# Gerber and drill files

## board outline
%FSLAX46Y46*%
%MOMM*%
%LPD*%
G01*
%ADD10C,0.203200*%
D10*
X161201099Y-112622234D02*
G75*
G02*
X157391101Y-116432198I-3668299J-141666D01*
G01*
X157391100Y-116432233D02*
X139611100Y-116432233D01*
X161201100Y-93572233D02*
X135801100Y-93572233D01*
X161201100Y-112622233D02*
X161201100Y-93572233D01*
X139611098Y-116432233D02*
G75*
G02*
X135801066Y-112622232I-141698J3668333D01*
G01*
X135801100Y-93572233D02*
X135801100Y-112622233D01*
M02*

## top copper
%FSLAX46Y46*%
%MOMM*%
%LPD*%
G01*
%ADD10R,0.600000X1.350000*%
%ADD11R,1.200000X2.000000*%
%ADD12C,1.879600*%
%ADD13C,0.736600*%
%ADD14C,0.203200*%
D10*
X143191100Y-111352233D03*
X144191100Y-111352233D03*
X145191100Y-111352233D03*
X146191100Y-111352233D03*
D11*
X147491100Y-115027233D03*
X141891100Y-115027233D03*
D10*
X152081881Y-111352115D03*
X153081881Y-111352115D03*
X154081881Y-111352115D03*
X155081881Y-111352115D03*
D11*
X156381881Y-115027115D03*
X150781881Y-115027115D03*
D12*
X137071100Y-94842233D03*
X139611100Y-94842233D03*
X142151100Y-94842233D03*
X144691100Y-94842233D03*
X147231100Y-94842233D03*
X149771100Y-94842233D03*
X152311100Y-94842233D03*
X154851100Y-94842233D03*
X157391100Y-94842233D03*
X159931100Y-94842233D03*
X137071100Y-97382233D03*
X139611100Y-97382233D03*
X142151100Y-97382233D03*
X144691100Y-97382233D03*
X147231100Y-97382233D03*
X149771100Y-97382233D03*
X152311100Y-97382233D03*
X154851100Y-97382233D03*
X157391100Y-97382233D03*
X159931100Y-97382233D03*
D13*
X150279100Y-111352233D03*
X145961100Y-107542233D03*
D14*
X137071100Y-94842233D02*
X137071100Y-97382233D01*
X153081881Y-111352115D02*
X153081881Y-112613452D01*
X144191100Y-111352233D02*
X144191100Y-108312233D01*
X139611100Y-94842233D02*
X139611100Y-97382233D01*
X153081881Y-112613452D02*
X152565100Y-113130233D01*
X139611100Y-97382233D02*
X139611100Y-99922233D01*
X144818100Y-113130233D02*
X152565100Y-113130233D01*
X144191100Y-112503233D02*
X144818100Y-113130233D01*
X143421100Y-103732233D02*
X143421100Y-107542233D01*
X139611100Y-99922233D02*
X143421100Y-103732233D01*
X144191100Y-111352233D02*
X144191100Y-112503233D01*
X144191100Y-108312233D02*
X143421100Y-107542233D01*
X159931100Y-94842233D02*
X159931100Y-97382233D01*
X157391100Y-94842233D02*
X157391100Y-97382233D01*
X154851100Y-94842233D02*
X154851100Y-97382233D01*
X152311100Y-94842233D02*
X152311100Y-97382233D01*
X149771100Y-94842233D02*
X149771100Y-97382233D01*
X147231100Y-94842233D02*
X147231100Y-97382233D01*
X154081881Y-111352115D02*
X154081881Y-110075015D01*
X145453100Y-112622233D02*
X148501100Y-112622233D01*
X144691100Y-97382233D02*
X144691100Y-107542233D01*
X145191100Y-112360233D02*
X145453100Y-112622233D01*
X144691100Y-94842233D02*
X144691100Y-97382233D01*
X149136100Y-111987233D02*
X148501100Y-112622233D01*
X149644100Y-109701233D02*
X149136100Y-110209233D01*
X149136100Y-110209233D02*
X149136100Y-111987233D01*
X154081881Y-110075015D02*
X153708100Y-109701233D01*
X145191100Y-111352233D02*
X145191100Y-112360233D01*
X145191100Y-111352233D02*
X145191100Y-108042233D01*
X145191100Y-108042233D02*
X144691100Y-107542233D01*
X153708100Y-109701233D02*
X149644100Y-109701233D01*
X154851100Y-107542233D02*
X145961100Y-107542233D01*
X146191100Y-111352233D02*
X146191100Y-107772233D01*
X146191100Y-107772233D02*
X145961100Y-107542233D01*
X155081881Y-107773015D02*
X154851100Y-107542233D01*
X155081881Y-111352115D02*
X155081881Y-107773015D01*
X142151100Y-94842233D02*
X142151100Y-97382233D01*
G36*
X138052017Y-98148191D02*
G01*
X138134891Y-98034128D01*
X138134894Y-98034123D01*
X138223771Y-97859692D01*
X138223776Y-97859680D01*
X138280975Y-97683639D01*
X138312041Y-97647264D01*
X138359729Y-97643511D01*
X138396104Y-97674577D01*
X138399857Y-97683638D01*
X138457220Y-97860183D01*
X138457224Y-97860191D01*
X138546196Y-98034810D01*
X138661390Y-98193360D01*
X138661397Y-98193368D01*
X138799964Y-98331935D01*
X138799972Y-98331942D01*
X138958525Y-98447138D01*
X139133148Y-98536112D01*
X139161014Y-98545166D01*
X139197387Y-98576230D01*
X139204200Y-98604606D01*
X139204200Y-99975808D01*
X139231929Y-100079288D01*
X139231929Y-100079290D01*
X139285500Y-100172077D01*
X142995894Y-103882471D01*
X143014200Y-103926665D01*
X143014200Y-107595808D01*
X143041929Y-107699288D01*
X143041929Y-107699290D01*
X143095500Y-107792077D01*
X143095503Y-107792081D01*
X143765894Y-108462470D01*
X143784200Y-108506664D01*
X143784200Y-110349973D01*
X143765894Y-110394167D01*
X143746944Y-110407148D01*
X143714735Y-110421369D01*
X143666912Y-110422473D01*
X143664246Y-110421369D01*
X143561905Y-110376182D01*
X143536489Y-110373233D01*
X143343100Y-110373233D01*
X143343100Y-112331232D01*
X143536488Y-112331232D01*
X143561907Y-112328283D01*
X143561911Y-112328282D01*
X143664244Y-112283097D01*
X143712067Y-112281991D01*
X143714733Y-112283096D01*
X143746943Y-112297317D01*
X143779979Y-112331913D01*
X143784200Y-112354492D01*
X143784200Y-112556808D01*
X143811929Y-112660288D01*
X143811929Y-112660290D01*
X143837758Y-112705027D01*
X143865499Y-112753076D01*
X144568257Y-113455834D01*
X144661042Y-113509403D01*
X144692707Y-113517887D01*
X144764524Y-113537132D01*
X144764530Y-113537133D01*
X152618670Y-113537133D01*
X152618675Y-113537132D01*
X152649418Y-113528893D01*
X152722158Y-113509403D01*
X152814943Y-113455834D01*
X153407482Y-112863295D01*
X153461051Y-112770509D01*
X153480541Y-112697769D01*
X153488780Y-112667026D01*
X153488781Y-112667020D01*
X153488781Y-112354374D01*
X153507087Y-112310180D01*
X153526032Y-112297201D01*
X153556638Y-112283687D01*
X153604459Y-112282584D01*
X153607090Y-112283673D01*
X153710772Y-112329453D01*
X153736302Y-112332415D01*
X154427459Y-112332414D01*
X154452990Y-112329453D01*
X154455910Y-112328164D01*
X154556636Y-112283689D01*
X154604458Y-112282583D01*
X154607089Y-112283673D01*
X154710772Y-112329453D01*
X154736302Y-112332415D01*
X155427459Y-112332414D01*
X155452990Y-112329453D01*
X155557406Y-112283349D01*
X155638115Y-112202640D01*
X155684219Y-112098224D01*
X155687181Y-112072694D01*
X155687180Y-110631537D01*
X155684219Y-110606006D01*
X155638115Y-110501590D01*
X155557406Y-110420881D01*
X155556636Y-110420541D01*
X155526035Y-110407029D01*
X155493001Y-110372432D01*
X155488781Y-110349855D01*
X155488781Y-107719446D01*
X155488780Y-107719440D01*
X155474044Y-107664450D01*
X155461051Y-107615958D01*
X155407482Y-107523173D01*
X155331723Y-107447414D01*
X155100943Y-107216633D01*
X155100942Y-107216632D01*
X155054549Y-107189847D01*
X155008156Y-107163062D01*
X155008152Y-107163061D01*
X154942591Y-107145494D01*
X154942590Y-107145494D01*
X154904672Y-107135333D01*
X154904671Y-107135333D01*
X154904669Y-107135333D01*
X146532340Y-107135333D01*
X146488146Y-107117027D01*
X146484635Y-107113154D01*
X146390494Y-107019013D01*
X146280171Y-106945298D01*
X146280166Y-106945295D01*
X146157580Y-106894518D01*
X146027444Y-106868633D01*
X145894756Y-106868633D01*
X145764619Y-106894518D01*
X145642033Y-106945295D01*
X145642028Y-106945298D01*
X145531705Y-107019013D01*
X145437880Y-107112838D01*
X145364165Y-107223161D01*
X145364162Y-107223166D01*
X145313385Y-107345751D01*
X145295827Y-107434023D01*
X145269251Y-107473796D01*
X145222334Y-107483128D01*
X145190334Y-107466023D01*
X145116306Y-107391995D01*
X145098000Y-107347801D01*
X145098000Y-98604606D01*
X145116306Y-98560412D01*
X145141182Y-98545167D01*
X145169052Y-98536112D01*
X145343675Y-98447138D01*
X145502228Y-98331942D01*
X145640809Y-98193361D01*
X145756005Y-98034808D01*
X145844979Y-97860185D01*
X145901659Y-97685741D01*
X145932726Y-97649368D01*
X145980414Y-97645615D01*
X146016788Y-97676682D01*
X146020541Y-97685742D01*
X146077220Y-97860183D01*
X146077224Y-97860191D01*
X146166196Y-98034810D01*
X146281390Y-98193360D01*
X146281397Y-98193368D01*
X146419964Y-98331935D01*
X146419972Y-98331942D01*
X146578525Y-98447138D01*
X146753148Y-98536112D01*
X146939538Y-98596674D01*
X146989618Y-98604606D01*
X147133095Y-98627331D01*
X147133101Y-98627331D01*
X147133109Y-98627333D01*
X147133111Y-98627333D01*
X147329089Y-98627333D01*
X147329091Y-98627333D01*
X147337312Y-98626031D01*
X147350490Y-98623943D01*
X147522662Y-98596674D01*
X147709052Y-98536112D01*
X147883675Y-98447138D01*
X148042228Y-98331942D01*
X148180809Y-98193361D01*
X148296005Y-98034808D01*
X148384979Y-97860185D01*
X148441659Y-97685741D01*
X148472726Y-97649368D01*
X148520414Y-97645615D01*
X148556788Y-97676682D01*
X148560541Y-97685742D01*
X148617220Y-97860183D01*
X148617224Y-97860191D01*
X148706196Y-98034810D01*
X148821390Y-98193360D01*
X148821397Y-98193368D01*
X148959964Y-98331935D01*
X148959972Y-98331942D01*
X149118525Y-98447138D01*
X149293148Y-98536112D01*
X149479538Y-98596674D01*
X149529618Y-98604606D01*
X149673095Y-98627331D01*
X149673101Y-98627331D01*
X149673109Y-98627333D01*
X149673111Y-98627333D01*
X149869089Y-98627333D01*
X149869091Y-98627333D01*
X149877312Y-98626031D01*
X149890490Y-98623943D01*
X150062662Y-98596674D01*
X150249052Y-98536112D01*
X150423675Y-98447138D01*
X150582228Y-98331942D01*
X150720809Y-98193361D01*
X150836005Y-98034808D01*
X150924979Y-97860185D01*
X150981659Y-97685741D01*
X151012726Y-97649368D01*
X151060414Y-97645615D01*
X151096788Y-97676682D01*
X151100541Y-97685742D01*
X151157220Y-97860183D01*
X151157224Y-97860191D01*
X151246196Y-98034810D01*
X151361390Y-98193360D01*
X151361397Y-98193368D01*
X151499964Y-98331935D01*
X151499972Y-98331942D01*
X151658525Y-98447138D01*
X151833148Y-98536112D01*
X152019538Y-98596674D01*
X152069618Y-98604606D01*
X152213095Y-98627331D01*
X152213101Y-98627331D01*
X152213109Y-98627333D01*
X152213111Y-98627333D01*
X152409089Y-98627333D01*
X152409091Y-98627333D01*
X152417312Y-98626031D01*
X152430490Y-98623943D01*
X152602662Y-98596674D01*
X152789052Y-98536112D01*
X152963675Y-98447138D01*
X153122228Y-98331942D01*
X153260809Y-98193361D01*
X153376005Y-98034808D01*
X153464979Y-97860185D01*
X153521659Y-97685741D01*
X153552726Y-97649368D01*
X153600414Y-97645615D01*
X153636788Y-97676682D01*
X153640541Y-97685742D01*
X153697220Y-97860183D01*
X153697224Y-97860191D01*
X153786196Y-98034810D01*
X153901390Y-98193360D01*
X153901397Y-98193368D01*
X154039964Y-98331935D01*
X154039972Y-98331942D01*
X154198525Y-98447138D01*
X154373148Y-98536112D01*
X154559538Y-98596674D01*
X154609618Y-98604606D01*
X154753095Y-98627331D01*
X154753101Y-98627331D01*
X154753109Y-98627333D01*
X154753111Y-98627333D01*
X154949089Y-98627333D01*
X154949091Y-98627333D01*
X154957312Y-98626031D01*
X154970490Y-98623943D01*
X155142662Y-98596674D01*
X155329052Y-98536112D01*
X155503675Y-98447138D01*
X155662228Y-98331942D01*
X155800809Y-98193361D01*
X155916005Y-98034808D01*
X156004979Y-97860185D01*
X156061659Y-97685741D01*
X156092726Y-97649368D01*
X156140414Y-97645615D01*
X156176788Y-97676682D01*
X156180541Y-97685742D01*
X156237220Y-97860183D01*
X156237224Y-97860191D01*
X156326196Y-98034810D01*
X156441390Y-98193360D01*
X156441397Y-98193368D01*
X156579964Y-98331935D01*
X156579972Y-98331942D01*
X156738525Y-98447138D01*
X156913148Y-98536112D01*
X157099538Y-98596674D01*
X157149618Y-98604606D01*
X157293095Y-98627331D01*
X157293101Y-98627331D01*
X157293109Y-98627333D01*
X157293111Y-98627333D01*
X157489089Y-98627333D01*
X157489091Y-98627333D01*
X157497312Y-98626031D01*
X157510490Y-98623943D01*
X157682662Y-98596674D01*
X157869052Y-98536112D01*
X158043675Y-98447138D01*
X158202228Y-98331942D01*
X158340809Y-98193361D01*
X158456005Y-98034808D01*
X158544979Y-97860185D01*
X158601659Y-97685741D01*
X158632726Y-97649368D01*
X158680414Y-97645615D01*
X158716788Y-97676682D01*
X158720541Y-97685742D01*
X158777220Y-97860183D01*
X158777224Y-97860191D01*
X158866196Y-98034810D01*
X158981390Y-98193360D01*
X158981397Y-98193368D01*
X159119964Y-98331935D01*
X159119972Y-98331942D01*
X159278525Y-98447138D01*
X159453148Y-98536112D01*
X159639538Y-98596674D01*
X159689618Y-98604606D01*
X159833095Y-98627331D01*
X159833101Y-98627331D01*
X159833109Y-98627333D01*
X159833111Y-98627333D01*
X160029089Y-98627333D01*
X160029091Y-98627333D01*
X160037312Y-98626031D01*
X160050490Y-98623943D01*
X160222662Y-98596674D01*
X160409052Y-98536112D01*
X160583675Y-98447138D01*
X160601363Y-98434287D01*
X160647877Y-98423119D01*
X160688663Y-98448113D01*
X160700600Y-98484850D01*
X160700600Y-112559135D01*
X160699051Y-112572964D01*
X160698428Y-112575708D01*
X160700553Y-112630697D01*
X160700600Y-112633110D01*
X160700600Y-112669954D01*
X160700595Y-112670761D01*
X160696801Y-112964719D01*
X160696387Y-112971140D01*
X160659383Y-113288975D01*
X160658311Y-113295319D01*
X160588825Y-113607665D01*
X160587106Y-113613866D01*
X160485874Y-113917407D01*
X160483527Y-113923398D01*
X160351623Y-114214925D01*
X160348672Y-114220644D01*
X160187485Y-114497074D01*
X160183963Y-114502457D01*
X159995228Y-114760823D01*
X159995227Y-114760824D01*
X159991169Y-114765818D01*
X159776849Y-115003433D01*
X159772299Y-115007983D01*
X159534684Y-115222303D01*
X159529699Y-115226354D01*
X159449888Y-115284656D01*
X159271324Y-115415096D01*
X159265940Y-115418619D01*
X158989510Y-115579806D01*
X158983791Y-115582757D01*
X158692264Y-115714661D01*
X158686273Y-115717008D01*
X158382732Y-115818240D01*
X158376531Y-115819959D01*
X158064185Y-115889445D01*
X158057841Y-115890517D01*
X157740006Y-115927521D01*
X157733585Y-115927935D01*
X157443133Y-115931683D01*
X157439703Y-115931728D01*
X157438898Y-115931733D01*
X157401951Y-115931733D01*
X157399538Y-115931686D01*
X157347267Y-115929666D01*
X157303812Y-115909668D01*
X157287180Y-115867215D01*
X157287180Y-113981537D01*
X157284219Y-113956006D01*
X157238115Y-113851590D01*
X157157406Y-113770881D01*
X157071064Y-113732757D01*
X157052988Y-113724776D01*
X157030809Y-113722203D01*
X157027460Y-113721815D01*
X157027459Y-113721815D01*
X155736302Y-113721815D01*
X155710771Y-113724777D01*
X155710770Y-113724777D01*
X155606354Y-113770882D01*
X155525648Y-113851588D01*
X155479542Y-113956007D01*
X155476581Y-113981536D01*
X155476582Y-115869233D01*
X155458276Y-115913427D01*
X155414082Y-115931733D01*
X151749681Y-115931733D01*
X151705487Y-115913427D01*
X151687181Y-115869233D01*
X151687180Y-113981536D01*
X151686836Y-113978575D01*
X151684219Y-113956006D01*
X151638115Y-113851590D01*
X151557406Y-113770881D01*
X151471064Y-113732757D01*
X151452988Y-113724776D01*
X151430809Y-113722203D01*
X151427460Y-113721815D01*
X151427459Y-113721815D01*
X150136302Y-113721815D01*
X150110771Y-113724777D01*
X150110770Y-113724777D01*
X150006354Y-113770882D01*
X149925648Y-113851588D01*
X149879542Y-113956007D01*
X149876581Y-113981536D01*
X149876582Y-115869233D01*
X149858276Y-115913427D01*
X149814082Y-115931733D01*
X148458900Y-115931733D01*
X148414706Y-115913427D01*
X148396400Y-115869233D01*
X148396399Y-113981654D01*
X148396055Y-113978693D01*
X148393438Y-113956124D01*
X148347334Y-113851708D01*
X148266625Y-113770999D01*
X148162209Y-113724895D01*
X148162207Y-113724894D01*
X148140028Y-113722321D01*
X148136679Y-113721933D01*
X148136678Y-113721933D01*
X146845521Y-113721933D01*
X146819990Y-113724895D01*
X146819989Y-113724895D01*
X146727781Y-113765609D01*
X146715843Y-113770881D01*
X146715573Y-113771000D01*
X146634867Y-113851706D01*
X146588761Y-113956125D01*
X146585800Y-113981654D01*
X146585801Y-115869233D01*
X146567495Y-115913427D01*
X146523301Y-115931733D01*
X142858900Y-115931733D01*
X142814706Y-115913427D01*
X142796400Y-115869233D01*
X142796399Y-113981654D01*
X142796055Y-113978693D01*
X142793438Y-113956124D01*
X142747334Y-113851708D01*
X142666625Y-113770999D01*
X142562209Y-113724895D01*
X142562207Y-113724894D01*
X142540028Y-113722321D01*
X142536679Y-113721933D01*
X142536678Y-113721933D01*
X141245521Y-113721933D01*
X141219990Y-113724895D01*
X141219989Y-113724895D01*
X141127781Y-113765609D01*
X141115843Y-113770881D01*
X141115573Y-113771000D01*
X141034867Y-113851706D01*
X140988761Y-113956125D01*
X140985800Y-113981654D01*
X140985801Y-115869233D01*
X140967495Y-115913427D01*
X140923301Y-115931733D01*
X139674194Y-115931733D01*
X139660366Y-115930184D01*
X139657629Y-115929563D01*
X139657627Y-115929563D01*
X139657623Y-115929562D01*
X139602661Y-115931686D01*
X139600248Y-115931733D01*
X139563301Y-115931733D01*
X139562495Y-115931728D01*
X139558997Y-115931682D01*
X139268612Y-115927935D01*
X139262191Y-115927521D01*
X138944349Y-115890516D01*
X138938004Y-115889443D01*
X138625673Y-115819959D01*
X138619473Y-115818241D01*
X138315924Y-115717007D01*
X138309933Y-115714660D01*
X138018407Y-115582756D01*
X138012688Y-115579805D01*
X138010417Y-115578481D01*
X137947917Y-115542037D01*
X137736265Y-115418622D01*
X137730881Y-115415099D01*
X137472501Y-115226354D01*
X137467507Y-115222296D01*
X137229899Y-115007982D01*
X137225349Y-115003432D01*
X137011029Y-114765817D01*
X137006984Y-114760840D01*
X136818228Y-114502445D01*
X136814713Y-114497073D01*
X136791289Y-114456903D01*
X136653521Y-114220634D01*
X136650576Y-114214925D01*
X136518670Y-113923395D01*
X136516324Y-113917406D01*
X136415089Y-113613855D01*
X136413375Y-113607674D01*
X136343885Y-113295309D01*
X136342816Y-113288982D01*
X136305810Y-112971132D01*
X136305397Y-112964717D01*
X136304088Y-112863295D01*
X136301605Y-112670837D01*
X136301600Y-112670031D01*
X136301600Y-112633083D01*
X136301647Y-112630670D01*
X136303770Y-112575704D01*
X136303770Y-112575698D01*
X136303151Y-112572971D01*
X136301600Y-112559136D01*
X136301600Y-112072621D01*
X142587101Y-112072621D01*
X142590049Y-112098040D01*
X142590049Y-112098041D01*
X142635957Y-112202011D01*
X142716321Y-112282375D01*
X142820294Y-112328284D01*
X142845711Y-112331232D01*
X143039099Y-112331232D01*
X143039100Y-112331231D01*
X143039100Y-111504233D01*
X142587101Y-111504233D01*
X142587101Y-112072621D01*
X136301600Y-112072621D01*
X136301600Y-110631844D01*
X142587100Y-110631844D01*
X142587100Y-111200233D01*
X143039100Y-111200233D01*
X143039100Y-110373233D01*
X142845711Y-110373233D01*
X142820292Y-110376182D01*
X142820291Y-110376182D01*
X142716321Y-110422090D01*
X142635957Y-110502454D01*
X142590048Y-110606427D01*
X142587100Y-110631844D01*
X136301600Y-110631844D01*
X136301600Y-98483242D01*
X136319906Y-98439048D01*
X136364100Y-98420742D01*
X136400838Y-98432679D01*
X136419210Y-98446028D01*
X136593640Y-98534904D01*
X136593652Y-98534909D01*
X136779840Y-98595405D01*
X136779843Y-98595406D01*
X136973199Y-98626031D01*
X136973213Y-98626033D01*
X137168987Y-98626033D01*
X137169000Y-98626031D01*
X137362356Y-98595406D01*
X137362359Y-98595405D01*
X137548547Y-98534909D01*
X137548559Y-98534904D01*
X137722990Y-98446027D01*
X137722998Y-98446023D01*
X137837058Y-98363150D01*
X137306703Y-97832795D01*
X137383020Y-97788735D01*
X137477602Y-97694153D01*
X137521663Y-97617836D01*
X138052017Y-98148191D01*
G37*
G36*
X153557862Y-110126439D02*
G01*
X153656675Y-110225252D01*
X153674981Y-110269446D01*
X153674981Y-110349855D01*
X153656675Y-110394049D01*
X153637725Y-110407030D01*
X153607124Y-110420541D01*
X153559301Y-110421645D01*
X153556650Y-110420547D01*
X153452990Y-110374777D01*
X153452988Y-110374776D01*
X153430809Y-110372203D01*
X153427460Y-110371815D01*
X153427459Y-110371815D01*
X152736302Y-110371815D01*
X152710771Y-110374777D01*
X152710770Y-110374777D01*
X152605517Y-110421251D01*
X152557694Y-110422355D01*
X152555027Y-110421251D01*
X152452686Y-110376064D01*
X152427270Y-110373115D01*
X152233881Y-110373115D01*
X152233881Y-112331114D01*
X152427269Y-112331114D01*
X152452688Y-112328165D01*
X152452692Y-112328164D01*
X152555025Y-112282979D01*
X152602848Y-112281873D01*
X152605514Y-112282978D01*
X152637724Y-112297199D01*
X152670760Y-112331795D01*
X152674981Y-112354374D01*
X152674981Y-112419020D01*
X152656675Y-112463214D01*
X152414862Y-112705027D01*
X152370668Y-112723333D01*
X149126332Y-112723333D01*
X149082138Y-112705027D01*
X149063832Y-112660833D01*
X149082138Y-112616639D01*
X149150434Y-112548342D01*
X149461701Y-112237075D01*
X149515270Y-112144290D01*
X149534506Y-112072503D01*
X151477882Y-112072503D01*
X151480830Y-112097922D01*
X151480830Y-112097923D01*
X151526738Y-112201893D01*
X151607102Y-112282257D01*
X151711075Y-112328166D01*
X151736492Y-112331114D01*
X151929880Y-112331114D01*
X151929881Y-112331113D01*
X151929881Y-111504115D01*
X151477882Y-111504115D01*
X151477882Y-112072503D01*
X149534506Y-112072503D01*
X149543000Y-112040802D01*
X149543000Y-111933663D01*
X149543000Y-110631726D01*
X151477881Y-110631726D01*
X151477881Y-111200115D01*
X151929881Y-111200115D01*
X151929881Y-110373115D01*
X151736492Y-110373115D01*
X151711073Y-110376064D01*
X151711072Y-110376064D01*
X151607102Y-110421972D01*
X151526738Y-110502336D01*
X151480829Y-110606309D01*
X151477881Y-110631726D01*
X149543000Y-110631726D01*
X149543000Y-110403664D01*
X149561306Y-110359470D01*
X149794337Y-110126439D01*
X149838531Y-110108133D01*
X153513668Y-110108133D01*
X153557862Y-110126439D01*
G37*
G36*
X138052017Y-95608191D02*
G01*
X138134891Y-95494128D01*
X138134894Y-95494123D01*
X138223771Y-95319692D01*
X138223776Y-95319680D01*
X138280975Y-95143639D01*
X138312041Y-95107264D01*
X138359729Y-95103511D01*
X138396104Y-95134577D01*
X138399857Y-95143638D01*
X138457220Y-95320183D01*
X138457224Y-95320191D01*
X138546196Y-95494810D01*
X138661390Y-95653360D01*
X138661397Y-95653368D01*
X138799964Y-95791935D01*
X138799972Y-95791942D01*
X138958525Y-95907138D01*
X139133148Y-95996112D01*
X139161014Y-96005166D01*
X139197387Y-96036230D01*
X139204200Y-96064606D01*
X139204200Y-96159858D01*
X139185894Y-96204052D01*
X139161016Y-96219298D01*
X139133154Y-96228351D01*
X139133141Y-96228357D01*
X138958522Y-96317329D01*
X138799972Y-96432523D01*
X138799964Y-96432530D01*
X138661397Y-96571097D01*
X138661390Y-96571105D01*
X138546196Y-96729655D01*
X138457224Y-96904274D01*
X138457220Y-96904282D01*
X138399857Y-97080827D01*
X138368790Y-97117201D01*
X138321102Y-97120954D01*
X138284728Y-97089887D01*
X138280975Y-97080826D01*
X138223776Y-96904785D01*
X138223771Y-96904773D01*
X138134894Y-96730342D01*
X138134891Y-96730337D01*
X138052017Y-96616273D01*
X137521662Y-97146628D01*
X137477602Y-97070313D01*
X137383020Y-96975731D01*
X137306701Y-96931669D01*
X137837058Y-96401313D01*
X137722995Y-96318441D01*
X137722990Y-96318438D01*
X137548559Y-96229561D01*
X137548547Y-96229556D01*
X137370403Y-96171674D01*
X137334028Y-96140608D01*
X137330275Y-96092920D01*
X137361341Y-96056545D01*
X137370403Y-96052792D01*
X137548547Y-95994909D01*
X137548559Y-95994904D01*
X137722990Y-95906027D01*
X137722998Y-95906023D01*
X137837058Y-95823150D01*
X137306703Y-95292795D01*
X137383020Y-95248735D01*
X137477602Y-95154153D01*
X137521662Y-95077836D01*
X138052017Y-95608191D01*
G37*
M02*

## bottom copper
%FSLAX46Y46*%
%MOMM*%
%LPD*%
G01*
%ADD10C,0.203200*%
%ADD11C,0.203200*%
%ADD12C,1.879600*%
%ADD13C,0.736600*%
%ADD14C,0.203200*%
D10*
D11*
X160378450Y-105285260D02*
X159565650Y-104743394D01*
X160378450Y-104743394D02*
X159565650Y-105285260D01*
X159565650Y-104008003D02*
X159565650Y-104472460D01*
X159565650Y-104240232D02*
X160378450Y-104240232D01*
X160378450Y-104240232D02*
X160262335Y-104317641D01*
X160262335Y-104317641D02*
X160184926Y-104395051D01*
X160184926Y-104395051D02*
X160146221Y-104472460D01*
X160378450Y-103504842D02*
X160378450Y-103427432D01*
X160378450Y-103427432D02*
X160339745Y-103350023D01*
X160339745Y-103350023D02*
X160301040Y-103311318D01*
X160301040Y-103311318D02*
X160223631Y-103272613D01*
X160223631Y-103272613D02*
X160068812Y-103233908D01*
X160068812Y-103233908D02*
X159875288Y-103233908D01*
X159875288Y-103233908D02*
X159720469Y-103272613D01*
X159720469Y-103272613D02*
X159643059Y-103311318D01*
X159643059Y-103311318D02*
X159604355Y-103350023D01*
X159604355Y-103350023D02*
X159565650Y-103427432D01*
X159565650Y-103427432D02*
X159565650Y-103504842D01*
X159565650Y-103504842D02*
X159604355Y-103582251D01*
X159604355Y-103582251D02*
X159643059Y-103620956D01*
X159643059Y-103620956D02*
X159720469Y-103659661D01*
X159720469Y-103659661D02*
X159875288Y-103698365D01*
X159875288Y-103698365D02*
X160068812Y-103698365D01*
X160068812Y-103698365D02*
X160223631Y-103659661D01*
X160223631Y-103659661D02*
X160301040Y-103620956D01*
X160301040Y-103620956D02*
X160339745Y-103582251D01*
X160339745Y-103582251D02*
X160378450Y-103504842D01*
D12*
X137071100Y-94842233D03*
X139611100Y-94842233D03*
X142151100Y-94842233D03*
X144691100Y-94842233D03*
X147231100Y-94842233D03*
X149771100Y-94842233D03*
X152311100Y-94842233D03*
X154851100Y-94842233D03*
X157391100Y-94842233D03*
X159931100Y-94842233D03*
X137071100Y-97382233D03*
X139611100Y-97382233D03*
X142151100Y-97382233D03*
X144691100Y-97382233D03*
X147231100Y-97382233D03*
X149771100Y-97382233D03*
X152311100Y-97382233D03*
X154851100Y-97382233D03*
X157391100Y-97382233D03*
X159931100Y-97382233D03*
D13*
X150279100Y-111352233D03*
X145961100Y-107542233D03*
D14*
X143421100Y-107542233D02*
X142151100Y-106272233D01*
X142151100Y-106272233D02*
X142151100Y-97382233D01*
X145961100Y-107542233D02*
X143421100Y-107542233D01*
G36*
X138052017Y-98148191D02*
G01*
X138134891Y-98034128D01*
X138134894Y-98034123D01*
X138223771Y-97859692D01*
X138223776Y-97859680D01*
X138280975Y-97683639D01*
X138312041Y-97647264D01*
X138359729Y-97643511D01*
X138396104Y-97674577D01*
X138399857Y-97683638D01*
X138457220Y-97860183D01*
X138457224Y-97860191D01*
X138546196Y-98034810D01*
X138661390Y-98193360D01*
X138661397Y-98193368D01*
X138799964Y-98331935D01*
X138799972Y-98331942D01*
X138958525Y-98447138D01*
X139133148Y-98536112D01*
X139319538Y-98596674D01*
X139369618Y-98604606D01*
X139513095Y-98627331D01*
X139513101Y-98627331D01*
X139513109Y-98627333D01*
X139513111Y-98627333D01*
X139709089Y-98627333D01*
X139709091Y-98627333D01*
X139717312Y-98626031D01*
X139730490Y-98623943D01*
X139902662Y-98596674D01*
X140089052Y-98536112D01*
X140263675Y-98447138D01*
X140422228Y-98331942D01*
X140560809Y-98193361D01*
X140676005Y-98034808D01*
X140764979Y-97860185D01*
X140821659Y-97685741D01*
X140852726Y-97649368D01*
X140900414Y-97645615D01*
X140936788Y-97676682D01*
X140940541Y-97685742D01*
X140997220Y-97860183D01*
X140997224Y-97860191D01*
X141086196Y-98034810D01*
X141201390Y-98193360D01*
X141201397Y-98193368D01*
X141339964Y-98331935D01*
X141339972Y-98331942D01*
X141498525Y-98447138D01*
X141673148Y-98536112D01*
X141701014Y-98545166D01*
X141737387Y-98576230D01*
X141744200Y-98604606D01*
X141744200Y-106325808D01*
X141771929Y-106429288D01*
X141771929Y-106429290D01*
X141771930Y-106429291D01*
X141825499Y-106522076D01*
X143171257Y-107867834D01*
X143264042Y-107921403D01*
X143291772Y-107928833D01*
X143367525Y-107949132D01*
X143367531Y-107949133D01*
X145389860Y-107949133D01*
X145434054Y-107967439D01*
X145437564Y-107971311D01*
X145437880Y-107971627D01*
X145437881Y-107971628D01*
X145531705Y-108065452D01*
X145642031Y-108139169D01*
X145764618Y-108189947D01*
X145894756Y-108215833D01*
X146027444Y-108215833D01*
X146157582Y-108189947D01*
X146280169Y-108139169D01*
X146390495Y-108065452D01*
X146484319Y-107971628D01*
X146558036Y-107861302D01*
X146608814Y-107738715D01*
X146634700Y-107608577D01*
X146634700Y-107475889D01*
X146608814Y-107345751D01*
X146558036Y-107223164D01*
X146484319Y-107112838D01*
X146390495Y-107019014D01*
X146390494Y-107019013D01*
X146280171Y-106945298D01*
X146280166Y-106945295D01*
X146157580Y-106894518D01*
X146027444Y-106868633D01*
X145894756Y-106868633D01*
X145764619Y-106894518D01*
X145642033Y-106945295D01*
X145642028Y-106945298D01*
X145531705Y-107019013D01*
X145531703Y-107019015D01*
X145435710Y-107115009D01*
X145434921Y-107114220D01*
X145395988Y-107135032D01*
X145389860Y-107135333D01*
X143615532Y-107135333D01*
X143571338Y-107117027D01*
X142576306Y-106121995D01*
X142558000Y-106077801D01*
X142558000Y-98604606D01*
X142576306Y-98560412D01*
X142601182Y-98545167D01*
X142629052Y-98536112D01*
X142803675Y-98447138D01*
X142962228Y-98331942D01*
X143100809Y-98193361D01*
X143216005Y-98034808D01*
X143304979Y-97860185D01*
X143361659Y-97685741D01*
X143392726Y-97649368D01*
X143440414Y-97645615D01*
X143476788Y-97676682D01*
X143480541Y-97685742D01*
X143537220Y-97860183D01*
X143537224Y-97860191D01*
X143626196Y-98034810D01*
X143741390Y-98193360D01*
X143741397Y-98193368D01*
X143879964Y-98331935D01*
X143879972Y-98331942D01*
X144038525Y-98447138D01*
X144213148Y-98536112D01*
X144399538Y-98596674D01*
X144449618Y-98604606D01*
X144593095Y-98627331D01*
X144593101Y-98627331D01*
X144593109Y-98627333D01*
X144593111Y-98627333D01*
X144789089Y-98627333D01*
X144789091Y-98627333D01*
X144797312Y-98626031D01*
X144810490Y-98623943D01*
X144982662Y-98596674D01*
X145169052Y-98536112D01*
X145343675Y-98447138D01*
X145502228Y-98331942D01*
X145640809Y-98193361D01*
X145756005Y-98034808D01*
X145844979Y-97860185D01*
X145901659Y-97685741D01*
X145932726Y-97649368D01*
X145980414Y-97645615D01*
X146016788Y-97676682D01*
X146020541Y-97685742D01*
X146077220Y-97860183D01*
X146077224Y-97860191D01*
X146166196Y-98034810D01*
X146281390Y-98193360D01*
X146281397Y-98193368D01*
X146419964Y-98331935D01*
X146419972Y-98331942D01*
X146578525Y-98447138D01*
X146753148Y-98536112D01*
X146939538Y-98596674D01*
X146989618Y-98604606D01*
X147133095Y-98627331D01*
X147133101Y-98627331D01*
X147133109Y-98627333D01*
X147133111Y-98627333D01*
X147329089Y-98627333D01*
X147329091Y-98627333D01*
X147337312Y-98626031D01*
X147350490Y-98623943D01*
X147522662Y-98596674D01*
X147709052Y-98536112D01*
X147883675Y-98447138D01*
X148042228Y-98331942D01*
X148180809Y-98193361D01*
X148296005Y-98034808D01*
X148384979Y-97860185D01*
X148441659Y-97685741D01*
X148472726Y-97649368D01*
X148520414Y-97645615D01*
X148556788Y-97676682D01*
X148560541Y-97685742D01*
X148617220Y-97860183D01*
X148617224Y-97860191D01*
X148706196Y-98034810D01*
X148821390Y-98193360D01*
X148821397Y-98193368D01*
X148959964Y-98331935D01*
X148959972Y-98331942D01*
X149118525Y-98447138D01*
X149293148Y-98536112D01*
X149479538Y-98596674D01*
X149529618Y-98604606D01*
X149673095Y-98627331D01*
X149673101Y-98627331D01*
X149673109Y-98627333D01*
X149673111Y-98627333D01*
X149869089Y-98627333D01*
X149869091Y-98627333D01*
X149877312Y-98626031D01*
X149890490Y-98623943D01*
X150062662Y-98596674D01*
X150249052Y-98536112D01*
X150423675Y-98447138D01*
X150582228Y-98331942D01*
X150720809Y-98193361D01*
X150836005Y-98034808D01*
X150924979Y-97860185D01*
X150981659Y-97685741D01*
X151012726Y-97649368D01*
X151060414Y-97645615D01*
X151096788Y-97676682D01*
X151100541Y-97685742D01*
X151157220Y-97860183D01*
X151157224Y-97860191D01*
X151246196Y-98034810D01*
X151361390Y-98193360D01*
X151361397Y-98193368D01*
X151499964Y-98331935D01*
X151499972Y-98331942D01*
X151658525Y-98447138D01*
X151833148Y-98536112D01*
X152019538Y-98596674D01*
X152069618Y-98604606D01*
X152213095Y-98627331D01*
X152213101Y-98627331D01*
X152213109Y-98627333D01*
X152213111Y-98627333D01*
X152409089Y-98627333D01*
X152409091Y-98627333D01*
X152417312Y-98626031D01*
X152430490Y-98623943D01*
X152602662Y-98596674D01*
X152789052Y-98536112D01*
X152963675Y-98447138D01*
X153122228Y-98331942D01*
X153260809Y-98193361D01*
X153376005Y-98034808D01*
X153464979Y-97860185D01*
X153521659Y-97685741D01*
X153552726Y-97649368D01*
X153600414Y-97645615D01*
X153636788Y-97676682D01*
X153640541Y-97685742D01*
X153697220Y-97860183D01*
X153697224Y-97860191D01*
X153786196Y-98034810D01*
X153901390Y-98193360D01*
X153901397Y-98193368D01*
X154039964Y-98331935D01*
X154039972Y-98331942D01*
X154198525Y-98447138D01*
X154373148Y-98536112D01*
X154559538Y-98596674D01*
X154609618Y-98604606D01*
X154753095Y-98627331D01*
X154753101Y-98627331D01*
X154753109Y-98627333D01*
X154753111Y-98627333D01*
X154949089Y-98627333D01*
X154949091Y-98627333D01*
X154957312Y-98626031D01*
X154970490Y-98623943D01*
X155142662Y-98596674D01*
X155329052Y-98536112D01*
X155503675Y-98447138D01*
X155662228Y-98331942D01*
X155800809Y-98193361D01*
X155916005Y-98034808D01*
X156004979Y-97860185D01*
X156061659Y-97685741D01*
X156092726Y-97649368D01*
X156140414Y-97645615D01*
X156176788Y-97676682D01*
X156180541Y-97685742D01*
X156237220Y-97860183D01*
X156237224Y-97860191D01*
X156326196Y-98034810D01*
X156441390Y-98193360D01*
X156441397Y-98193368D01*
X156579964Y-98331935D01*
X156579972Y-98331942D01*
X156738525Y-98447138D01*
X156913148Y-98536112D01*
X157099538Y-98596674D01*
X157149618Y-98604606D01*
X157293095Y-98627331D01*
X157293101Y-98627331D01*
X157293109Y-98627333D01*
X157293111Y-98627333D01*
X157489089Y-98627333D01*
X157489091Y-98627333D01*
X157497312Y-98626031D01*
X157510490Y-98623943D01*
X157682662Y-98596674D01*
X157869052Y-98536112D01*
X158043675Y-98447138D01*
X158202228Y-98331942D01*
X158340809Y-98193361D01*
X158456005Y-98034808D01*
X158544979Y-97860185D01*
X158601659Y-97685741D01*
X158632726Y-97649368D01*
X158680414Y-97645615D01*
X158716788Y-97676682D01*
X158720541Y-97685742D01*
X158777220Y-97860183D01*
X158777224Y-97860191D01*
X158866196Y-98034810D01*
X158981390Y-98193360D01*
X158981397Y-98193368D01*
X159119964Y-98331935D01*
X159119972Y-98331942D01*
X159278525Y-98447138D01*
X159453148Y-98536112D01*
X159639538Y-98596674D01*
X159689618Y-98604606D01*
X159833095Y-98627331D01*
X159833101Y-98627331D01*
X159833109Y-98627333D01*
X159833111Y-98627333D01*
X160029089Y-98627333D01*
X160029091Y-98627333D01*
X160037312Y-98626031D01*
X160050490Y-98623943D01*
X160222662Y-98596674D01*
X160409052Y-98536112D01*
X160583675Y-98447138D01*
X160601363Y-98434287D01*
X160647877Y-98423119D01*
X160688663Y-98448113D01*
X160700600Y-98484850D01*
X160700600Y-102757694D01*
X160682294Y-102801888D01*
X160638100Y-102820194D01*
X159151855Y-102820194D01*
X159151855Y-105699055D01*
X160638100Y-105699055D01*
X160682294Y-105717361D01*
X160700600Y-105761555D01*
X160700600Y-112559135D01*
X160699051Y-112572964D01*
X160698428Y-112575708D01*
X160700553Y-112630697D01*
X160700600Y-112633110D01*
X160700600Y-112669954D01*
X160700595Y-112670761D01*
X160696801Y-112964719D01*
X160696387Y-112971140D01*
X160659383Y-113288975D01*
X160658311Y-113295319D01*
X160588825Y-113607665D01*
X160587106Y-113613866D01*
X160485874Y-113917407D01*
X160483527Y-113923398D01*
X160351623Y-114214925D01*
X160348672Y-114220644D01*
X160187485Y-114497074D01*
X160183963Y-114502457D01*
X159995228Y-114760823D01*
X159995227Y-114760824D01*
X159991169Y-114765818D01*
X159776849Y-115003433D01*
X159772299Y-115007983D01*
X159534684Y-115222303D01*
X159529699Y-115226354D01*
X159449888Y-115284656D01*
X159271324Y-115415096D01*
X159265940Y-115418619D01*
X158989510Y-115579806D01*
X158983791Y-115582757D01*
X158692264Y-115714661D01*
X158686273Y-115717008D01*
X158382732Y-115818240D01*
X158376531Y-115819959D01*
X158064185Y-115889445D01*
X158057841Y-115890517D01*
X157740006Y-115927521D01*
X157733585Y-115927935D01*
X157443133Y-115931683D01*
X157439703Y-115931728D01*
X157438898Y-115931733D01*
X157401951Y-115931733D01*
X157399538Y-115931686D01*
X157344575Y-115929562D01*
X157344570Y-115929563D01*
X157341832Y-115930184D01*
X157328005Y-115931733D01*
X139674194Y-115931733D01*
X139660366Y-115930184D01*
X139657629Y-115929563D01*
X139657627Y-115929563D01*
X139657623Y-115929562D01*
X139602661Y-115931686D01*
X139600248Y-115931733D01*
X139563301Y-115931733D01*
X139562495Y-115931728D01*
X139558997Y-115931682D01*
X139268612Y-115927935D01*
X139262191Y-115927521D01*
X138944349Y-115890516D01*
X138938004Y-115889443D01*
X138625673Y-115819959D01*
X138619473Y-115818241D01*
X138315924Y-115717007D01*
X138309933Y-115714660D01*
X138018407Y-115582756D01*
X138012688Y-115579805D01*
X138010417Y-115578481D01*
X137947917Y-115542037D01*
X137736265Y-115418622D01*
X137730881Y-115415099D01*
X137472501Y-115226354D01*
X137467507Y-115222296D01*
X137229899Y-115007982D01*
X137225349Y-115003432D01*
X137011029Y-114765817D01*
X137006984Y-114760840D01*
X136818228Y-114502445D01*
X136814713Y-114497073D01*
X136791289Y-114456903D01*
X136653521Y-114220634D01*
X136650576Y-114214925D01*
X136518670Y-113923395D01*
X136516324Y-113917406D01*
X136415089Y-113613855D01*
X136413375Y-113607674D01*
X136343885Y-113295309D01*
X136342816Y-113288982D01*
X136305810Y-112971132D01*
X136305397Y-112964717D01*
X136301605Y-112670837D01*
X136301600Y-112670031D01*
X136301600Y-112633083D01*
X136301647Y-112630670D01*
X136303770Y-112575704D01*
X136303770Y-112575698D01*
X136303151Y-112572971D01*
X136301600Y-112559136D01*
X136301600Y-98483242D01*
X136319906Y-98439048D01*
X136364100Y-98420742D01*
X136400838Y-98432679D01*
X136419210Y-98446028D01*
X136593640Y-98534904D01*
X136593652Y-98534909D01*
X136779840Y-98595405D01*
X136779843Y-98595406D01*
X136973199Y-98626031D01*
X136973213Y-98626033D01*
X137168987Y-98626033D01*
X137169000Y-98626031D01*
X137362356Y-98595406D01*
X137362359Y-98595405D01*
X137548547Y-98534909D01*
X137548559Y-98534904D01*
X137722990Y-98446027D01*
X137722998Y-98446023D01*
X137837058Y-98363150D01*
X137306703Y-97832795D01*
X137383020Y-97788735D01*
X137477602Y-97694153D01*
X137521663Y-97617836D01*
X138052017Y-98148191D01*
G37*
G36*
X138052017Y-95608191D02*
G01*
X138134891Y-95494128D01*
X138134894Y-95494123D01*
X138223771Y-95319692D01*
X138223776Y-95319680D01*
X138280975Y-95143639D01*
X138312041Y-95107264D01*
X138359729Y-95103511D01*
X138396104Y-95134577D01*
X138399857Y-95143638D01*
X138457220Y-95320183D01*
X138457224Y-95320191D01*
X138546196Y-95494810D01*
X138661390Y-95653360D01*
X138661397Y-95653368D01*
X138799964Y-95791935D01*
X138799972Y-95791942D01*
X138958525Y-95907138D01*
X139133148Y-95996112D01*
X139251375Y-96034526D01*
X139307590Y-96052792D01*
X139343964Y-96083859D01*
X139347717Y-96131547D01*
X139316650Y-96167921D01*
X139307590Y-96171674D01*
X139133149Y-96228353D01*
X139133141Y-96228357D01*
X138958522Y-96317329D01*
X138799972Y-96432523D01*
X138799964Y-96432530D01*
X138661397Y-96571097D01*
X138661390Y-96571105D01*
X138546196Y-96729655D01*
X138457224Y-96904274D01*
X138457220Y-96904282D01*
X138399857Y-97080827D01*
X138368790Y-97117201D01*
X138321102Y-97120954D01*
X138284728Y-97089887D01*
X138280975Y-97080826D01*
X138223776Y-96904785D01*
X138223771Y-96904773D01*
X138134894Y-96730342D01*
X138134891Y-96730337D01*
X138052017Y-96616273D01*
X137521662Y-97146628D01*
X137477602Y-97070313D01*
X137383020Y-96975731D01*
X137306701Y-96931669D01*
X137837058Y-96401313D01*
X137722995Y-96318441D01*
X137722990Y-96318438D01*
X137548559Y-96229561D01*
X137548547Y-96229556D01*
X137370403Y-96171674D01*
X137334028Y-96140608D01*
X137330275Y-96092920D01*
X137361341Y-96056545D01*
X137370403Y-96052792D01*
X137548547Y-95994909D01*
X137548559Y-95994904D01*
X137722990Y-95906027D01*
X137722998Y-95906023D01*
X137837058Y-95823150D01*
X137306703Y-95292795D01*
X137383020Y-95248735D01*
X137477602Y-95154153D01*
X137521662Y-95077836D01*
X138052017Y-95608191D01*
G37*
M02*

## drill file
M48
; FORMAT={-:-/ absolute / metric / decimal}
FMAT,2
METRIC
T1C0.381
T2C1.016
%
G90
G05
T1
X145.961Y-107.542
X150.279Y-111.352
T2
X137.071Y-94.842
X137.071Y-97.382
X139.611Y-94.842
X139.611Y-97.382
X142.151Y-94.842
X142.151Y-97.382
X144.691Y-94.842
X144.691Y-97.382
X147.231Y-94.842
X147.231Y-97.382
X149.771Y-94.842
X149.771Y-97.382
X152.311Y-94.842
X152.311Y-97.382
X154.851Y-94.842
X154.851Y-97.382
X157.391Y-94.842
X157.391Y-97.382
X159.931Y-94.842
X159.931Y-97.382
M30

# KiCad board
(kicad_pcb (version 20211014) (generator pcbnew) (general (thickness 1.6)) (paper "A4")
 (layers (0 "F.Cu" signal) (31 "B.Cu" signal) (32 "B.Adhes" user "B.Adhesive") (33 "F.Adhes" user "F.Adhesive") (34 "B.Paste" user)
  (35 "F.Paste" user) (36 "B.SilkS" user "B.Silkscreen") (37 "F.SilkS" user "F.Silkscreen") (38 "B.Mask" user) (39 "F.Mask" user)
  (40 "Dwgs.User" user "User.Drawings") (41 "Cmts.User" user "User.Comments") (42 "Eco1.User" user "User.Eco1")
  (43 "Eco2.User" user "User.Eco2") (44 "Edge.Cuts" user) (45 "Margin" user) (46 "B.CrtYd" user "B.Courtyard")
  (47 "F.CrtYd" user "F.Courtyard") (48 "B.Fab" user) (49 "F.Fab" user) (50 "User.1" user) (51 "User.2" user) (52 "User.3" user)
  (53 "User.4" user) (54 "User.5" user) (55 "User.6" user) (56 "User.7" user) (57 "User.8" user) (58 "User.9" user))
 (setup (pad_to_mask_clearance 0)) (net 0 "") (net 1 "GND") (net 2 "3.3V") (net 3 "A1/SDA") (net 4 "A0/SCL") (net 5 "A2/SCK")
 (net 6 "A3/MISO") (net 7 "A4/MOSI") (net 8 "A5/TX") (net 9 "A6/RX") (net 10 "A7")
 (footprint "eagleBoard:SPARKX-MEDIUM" (layer "F.Cu") (at 138.3411 108.812233 90)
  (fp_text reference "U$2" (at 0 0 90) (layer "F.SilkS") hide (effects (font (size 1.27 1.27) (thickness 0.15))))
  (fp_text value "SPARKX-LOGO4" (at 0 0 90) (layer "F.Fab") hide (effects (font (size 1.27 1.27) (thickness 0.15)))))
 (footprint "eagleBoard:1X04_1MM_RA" (layer "F.Cu") (at 144.6911 111.352233)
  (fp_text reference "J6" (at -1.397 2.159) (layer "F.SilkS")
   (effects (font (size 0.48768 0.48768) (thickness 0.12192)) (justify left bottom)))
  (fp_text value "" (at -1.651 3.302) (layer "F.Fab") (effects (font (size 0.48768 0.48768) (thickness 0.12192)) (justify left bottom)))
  (pad "1" smd rect (at -1.5 0) (size 0.6 1.35) (layers "F.Cu" "F.Paste" "F.Mask") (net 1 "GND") (solder_mask_margin 0.1016))
  (pad "2" smd rect (at -0.5 0) (size 0.6 1.35) (layers "F.Cu" "F.Paste" "F.Mask") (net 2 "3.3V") (solder_mask_margin 0.1016))
  (pad "3" smd rect (at 0.5 0) (size 0.6 1.35) (layers "F.Cu" "F.Paste" "F.Mask") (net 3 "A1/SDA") (solder_mask_margin 0.1016))
  (pad "4" smd rect (at 1.5 0) (size 0.6 1.35) (layers "F.Cu" "F.Paste" "F.Mask") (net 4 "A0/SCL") (solder_mask_margin 0.1016))
  (pad "NC1" smd rect (at 2.8 3.675) (size 1.2 2) (layers "F.Cu" "F.Paste" "F.Mask") (solder_mask_margin 0.1016))
  (pad "NC2" smd rect (at -2.8 3.675) (size 1.2 2) (layers "F.Cu" "F.Paste" "F.Mask") (solder_mask_margin 0.1016)))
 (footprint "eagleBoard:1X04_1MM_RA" (layer "F.Cu") (at 153.581881 111.352115)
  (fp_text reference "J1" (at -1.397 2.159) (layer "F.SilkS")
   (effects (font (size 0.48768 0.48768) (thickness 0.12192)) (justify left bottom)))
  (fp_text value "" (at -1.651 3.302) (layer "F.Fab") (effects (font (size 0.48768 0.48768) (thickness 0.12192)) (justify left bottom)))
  (pad "1" smd rect (at -1.5 0) (size 0.6 1.35) (layers "F.Cu" "F.Paste" "F.Mask") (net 1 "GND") (solder_mask_margin 0.1016))
  (pad "2" smd rect (at -0.5 0) (size 0.6 1.35) (layers "F.Cu" "F.Paste" "F.Mask") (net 2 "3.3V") (solder_mask_margin 0.1016))
  (pad "3" smd rect (at 0.5 0) (size 0.6 1.35) (layers "F.Cu" "F.Paste" "F.Mask") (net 3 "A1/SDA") (solder_mask_margin 0.1016))
  (pad "4" smd rect (at 1.5 0) (size 0.6 1.35) (layers "F.Cu" "F.Paste" "F.Mask") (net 4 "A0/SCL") (solder_mask_margin 0.1016))
  (pad "NC1" smd rect (at 2.8 3.675) (size 1.2 2) (layers "F.Cu" "F.Paste" "F.Mask") (solder_mask_margin 0.1016))
  (pad "NC2" smd rect (at -2.8 3.675) (size 1.2 2) (layers "F.Cu" "F.Paste" "F.Mask") (solder_mask_margin 0.1016)))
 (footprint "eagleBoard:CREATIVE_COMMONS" (layer "F.Cu") (at 126.9111 140.562233)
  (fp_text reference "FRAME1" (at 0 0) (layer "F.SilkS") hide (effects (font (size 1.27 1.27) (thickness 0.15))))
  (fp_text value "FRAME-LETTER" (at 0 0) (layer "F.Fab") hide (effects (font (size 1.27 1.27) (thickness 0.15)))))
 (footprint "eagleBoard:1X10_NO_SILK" (layer "F.Cu") (at 137.0711 94.842233)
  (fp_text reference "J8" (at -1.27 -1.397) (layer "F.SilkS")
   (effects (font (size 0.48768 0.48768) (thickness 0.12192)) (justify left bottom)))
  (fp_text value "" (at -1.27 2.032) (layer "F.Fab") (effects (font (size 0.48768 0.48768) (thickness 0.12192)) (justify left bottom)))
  (pad "1" thru_hole circle (at 0 0 90) (size 1.8796 1.8796) (drill 1.016) (layers *.Cu *.Mask) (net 1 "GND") (solder_mask_margin 0.1016))
  (pad "2" thru_hole circle (at 2.54 0 90) (size 1.8796 1.8796) (drill 1.016) (layers *.Cu *.Mask) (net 2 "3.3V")
   (solder_mask_margin 0.1016))
  (pad "3" thru_hole circle (at 5.08 0 90) (size 1.8796 1.8796) (drill 1.016) (layers *.Cu *.Mask) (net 4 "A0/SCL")
   (solder_mask_margin 0.1016))
  (pad "4" thru_hole circle (at 7.62 0 90) (size 1.8796 1.8796) (drill 1.016) (layers *.Cu *.Mask) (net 3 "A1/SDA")
   (solder_mask_margin 0.1016))
  (pad "5" thru_hole circle (at 10.16 0 90) (size 1.8796 1.8796) (drill 1.016) (layers *.Cu *.Mask) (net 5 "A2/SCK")
   (solder_mask_margin 0.1016))
  (pad "6" thru_hole circle (at 12.7 0 90) (size 1.8796 1.8796) (drill 1.016) (layers *.Cu *.Mask) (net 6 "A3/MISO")
   (solder_mask_margin 0.1016))
  (pad "7" thru_hole circle (at 15.24 0 90) (size 1.8796 1.8796) (drill 1.016) (layers *.Cu *.Mask) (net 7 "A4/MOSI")
   (solder_mask_margin 0.1016))
  (pad "8" thru_hole circle (at 17.78 0 90) (size 1.8796 1.8796) (drill 1.016) (layers *.Cu *.Mask) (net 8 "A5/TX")
   (solder_mask_margin 0.1016))
  (pad "9" thru_hole circle (at 20.32 0 90) (size 1.8796 1.8796) (drill 1.016) (layers *.Cu *.Mask) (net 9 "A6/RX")
   (solder_mask_margin 0.1016))
  (pad "10" thru_hole circle (at 22.86 0 90) (size 1.8796 1.8796) (drill 1.016) (layers *.Cu *.Mask) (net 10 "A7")
   (solder_mask_margin 0.1016)))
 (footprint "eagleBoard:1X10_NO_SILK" (layer "F.Cu") (at 137.0711 97.382233)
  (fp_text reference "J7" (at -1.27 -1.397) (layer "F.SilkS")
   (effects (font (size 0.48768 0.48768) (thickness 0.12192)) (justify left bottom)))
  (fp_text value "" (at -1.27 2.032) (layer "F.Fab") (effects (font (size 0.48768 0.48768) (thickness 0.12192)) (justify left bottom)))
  (pad "1" thru_hole circle (at 0 0 90) (size 1.8796 1.8796) (drill 1.016) (layers *.Cu *.Mask) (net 1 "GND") (solder_mask_margin 0.1016))
  (pad "2" thru_hole circle (at 2.54 0 90) (size 1.8796 1.8796) (drill 1.016) (layers *.Cu *.Mask) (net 2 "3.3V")
   (solder_mask_margin 0.1016))
  (pad "3" thru_hole circle (at 5.08 0 90) (size 1.8796 1.8796) (drill 1.016) (layers *.Cu *.Mask) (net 4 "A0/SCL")
   (solder_mask_margin 0.1016))
  (pad "4" thru_hole circle (at 7.62 0 90) (size 1.8796 1.8796) (drill 1.016) (layers *.Cu *.Mask) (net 3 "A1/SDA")
   (solder_mask_margin 0.1016))
  (pad "5" thru_hole circle (at 10.16 0 90) (size 1.8796 1.8796) (drill 1.016) (layers *.Cu *.Mask) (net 5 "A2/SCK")
   (solder_mask_margin 0.1016))
  (pad "6" thru_hole circle (at 12.7 0 90) (size 1.8796 1.8796) (drill 1.016) (layers *.Cu *.Mask) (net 6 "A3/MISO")
   (solder_mask_margin 0.1016))
  (pad "7" thru_hole circle (at 15.24 0 90) (size 1.8796 1.8796) (drill 1.016) (layers *.Cu *.Mask) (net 7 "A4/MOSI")
   (solder_mask_margin 0.1016))
  (pad "8" thru_hole circle (at 17.78 0 90) (size 1.8796 1.8796) (drill 1.016) (layers *.Cu *.Mask) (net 8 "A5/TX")
   (solder_mask_margin 0.1016))
  (pad "9" thru_hole circle (at 20.32 0 90) (size 1.8796 1.8796) (drill 1.016) (layers *.Cu *.Mask) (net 9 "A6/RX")
   (solder_mask_margin 0.1016))
  (pad "10" thru_hole circle (at 22.86 0 90) (size 1.8796 1.8796) (drill 1.016) (layers *.Cu *.Mask) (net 10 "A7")
   (solder_mask_margin 0.1016)))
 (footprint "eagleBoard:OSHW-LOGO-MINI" (layer "B.Cu") (at 159.4231 112.114233 180)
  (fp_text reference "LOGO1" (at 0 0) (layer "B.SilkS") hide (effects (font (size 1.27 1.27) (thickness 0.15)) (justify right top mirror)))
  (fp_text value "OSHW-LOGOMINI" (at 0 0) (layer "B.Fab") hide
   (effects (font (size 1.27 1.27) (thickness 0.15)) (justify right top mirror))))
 (gr_arc (start 161.201099 112.622234) (mid 160.128599 115.359733) (end 157.3911 116.432233) (layer "Edge.Cuts") (width 0.2032))
 (gr_line (start 157.3911 116.432233) (end 139.6111 116.432233) (layer "Edge.Cuts") (width 0.2032))
 (gr_line (start 161.2011 93.572233) (end 135.8011 93.572233) (layer "Edge.Cuts") (width 0.2032))
 (gr_line (start 161.2011 112.622233) (end 161.2011 93.572233) (layer "Edge.Cuts") (width 0.2032))
 (gr_arc (start 139.611098 116.432233) (mid 136.8736 115.359732) (end 135.8011 112.622233) (layer "Edge.Cuts") (width 0.2032))
 (gr_line (start 135.8011 93.572233) (end 135.8011 112.622233) (layer "Edge.Cuts") (width 0.2032))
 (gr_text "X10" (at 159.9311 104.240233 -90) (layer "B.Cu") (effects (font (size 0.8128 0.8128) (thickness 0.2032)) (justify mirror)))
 (segment (start 137.0711 94.842233) (end 137.0711 97.382233) (width 0.2032) (layer "F.Cu") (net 1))
 (via (at 150.2791 111.352233) (size 0.7366) (drill 0.381) (layers "F.Cu" "B.Cu") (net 1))
 (segment (start 153.081881 111.352115) (end 153.081881 112.613452) (width 0.2032) (layer "F.Cu") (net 2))
 (segment (start 144.1911 111.352233) (end 144.1911 108.312233) (width 0.2032) (layer "F.Cu") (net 2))
 (segment (start 139.6111 94.842233) (end 139.6111 97.382233) (width 0.2032) (layer "F.Cu") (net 2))
 (segment (start 153.081881 112.613452) (end 152.5651 113.130233) (width 0.2032) (layer "F.Cu") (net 2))
 (segment (start 139.6111 97.382233) (end 139.6111 99.922233) (width 0.2032) (layer "F.Cu") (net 2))
 (segment (start 144.8181 113.130233) (end 152.5651 113.130233) (width 0.2032) (layer "F.Cu") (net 2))
 (segment (start 144.1911 112.503233) (end 144.8181 113.130233) (width 0.2032) (layer "F.Cu") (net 2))
 (segment (start 143.4211 103.732233) (end 143.4211 107.542233) (width 0.2032) (layer "F.Cu") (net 2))
 (segment (start 139.6111 99.922233) (end 143.4211 103.732233) (width 0.2032) (layer "F.Cu") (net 2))
 (segment (start 144.1911 111.352233) (end 144.1911 112.503233) (width 0.2032) (layer "F.Cu") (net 2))
 (segment (start 144.1911 108.312233) (end 143.4211 107.542233) (width 0.2032) (layer "F.Cu") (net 2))
 (segment (start 159.9311 94.842233) (end 159.9311 97.382233) (width 0.2032) (layer "F.Cu") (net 10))
 (segment (start 157.3911 94.842233) (end 157.3911 97.382233) (width 0.2032) (layer "F.Cu") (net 9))
 (segment (start 154.8511 94.842233) (end 154.8511 97.382233) (width 0.2032) (layer "F.Cu") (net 8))
 (segment (start 152.3111 94.842233) (end 152.3111 97.382233) (width 0.2032) (layer "F.Cu") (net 7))
 (segment (start 149.7711 94.842233) (end 149.7711 97.382233) (width 0.2032) (layer "F.Cu") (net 6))
 (segment (start 147.2311 94.842233) (end 147.2311 97.382233) (width 0.2032) (layer "F.Cu") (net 5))
 (segment (start 154.081881 111.352115) (end 154.081881 110.075015) (width 0.2032) (layer "F.Cu") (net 3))
 (segment (start 145.4531 112.622233) (end 148.5011 112.622233) (width 0.2032) (layer "F.Cu") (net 3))
 (segment (start 144.6911 97.382233) (end 144.6911 107.542233) (width 0.2032) (layer "F.Cu") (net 3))
 (segment (start 145.1911 112.360233) (end 145.4531 112.622233) (width 0.2032) (layer "F.Cu") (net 3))
 (segment (start 144.6911 94.842233) (end 144.6911 97.382233) (width 0.2032) (layer "F.Cu") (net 3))
 (segment (start 149.1361 111.987233) (end 148.5011 112.622233) (width 0.2032) (layer "F.Cu") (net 3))
 (segment (start 149.6441 109.701233) (end 149.1361 110.209233) (width 0.2032) (layer "F.Cu") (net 3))
 (segment (start 149.1361 110.209233) (end 149.1361 111.987233) (width 0.2032) (layer "F.Cu") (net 3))
 (segment (start 154.081881 110.075015) (end 153.7081 109.701233) (width 0.2032) (layer "F.Cu") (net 3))
 (segment (start 145.1911 111.352233) (end 145.1911 112.360233) (width 0.2032) (layer "F.Cu") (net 3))
 (segment (start 145.1911 111.352233) (end 145.1911 108.042233) (width 0.2032) (layer "F.Cu") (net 3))
 (segment (start 145.1911 108.042233) (end 144.6911 107.542233) (width 0.2032) (layer "F.Cu") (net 3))
 (segment (start 153.7081 109.701233) (end 149.6441 109.701233) (width 0.2032) (layer "F.Cu") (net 3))
 (segment (start 154.8511 107.542233) (end 145.9611 107.542233) (width 0.2032) (layer "F.Cu") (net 4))
 (segment (start 146.1911 111.352233) (end 146.1911 107.772233) (width 0.2032) (layer "F.Cu") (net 4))
 (segment (start 146.1911 107.772233) (end 145.9611 107.542233) (width 0.2032) (layer "F.Cu") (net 4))
 (segment (start 155.081881 107.773015) (end 154.8511 107.542233) (width 0.2032) (layer "F.Cu") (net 4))
 (segment (start 155.081881 111.352115) (end 155.081881 107.773015) (width 0.2032) (layer "F.Cu") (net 4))
 (segment (start 142.1511 94.842233) (end 142.1511 97.382233) (width 0.2032) (layer "F.Cu") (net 4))
 (via (at 145.9611 107.542233) (size 0.7366) (drill 0.381) (layers "F.Cu" "B.Cu") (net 4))
 (segment (start 143.4211 107.542233) (end 142.1511 106.272233) (width 0.2032) (layer "B.Cu") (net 4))
 (segment (start 142.1511 106.272233) (end 142.1511 97.382233) (width 0.2032) (layer "B.Cu") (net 4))
 (segment (start 145.9611 107.542233) (end 143.4211 107.542233) (width 0.2032) (layer "B.Cu") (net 4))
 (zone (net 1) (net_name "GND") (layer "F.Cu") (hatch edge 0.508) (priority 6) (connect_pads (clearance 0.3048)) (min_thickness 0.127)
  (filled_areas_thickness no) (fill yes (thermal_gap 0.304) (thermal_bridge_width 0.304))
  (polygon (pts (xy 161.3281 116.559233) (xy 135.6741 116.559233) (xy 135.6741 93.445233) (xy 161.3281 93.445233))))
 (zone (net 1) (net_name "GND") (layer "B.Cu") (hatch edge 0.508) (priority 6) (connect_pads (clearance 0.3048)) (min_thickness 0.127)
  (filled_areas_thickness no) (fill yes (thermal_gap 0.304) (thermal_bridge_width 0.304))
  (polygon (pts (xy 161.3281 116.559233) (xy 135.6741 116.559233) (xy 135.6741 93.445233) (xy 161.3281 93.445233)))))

